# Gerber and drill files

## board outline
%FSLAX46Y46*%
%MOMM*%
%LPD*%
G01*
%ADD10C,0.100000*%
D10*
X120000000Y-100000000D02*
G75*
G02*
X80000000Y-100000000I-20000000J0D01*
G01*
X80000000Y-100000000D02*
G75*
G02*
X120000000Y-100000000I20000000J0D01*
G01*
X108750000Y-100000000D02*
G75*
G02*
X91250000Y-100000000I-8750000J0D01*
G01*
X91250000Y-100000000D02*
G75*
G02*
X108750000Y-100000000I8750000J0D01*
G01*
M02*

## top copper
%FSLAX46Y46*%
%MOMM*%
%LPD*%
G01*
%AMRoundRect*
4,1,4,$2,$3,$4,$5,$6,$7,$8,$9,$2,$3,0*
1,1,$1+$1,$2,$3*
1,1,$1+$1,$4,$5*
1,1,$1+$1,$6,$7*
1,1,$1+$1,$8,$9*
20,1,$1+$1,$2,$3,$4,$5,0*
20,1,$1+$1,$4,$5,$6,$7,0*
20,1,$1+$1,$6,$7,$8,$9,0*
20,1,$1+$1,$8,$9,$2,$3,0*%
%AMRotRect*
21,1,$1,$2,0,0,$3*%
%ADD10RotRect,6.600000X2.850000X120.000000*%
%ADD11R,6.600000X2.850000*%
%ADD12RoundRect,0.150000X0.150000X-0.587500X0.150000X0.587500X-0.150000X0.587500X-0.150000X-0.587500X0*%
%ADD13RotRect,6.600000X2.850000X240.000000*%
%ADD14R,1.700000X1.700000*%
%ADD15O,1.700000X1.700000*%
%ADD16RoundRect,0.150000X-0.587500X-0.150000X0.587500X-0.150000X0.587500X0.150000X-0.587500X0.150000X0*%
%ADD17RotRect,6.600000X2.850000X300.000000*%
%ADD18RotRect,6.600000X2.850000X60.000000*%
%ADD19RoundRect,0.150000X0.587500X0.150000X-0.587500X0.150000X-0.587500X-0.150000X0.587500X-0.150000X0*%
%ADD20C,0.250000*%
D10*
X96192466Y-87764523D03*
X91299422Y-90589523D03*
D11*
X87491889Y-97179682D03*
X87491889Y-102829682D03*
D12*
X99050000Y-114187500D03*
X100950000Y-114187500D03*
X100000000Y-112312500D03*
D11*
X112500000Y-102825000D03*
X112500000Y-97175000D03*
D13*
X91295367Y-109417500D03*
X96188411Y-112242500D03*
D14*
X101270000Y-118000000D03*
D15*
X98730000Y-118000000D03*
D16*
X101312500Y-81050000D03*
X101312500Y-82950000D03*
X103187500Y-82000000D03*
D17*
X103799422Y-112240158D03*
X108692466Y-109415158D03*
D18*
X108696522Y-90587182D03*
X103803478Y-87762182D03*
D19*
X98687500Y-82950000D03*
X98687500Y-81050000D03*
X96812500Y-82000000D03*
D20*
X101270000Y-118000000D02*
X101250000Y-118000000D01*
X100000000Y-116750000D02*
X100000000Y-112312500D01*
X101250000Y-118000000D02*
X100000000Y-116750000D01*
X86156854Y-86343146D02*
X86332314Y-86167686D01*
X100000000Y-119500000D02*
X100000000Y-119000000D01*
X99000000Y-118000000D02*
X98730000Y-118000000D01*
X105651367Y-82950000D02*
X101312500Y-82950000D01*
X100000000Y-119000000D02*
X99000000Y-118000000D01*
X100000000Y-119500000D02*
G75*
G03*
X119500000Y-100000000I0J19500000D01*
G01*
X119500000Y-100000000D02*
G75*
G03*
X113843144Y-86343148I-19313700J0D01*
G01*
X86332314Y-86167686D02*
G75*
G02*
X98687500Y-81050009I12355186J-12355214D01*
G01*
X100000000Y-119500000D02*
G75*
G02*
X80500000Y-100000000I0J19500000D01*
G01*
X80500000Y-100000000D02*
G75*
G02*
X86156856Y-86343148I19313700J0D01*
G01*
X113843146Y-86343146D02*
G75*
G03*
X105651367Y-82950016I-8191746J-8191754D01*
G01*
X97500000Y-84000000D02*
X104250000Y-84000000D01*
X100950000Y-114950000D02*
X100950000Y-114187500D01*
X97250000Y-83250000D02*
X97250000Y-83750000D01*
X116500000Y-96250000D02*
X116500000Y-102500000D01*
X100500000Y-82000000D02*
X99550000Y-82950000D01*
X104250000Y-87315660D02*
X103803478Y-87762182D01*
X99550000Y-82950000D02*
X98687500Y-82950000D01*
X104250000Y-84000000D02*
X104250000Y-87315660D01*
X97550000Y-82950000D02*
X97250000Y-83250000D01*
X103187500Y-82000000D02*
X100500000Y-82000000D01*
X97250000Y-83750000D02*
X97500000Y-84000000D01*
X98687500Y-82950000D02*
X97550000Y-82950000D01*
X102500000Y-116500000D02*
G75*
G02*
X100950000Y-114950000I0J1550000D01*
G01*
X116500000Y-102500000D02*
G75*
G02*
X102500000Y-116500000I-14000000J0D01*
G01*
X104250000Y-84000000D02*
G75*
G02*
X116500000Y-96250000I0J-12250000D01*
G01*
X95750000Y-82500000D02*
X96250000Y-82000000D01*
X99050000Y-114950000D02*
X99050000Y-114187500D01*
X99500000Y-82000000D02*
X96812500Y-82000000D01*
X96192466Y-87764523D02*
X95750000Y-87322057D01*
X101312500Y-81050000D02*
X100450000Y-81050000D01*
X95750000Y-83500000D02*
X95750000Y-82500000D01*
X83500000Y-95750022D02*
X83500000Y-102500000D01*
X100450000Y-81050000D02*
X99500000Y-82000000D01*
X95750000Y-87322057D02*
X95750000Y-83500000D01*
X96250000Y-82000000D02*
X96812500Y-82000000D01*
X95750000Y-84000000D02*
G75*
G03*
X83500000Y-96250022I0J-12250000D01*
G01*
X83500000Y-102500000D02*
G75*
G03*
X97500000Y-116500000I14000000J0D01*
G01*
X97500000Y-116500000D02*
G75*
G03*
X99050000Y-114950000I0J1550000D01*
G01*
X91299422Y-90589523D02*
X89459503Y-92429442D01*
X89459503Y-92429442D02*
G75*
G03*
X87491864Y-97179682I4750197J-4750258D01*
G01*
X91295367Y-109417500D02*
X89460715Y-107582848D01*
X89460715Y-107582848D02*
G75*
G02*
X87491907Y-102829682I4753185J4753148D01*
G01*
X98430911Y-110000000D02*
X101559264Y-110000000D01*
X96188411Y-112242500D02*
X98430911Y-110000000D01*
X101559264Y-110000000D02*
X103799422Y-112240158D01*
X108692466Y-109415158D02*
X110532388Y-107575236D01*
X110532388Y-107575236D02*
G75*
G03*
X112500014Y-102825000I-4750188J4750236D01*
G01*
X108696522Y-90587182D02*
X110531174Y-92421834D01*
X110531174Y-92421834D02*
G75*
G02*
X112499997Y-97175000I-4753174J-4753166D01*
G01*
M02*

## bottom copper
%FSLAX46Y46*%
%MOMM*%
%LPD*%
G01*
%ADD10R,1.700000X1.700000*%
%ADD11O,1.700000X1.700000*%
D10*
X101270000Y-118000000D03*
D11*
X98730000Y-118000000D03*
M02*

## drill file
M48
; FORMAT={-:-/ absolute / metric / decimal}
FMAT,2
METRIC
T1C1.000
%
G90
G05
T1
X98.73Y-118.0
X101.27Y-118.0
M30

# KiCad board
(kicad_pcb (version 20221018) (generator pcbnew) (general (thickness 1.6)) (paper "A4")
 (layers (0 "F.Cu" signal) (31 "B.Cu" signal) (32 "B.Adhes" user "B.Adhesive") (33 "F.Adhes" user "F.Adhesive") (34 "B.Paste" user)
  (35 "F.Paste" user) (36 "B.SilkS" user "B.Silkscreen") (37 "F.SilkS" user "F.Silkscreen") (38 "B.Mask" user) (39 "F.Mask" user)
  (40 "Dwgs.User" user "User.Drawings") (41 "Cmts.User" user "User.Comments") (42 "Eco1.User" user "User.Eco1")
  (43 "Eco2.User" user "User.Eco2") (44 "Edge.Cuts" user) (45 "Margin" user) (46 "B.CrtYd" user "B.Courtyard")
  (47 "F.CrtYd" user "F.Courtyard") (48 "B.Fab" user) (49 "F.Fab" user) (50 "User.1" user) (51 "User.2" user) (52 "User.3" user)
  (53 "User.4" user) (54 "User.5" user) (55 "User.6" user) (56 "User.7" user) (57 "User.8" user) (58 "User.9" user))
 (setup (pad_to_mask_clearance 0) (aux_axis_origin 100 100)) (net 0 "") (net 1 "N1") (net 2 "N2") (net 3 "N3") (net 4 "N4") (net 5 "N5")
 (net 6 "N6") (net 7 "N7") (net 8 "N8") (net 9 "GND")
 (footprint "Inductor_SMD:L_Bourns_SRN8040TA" (layer "F.Cu") (at 93.745944 89.177023 -150)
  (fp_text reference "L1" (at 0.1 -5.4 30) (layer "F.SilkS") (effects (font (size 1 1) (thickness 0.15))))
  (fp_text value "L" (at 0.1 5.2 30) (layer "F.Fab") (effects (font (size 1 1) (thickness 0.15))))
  (pad "1" smd rect (at -2.825 0 120) (size 6.6 2.85) (layers "F.Cu" "F.Paste" "F.Mask") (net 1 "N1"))
  (pad "2" smd rect (at 2.825 0 120) (size 6.6 2.85) (layers "F.Cu" "F.Paste" "F.Mask") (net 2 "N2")))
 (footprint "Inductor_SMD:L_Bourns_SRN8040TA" (layer "F.Cu") (at 87.491889 100.004682 -90)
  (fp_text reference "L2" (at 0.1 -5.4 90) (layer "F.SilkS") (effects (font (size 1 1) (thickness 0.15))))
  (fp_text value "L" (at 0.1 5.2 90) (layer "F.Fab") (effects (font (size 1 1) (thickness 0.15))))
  (pad "1" smd rect (at -2.825 0 180) (size 6.6 2.85) (layers "F.Cu" "F.Paste" "F.Mask") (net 2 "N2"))
  (pad "2" smd rect (at 2.825 0 180) (size 6.6 2.85) (layers "F.Cu" "F.Paste" "F.Mask") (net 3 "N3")))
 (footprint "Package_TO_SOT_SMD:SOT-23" (layer "F.Cu") (at 100 113.25 90)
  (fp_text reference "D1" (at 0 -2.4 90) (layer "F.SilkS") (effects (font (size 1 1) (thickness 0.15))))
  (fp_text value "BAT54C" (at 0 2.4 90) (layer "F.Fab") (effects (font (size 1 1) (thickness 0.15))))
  (pad "1" smd roundrect (at -0.9375 -0.95 90) (size 1.475 0.6) (layers "F.Cu" "F.Paste" "F.Mask") (roundrect_rratio 0.25) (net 1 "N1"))
  (pad "2" smd roundrect (at -0.9375 0.95 90) (size 1.475 0.6) (layers "F.Cu" "F.Paste" "F.Mask") (roundrect_rratio 0.25) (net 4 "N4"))
  (pad "3" smd roundrect (at 0.9375 0 90) (size 1.475 0.6) (layers "F.Cu" "F.Paste" "F.Mask") (roundrect_rratio 0.25) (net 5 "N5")))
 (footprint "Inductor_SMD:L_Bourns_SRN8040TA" (layer "F.Cu") (at 112.5 100 90)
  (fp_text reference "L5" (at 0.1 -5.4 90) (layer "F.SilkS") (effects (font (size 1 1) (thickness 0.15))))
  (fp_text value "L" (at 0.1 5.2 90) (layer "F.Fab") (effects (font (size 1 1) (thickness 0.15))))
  (pad "1" smd rect (at -2.825 0) (size 6.6 2.85) (layers "F.Cu" "F.Paste" "F.Mask") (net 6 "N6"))
  (pad "2" smd rect (at 2.825 0) (size 6.6 2.85) (layers "F.Cu" "F.Paste" "F.Mask") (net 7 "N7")))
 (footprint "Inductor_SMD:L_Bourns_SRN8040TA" (layer "F.Cu") (at 93.741889 110.83 -30)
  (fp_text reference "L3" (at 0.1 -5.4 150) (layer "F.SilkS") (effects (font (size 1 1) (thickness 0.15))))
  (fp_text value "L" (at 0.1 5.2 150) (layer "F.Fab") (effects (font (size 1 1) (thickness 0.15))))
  (pad "1" smd rect (at -2.825 0 240) (size 6.6 2.85) (layers "F.Cu" "F.Paste" "F.Mask") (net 3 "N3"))
  (pad "2" smd rect (at 2.825 0 240) (size 6.6 2.85) (layers "F.Cu" "F.Paste" "F.Mask") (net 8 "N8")))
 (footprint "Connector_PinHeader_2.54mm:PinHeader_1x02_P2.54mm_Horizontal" (layer "F.Cu") (at 101.27 118 -90)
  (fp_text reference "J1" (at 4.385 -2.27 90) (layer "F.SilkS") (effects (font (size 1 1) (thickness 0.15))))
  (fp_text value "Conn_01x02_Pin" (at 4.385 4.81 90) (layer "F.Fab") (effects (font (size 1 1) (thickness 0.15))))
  (pad "1" thru_hole rect (at 0 0 270) (size 1.7 1.7) (drill 1) (layers "*.Cu" "*.Mask") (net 5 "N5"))
  (pad "2" thru_hole oval (at 0 2.54 270) (size 1.7 1.7) (drill 1) (layers "*.Cu" "*.Mask") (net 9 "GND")))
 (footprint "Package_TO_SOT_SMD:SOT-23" (layer "F.Cu") (at 102.25 82)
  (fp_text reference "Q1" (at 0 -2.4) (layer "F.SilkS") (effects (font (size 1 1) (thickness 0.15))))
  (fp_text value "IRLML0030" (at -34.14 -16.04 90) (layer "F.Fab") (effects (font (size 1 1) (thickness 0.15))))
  (pad "1" smd roundrect (at -0.9375 -0.95) (size 1.475 0.6) (layers "F.Cu" "F.Paste" "F.Mask") (roundrect_rratio 0.25) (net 1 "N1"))
  (pad "2" smd roundrect (at -0.9375 0.95) (size 1.475 0.6) (layers "F.Cu" "F.Paste" "F.Mask") (roundrect_rratio 0.25) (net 9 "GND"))
  (pad "3" smd roundrect (at 0.9375 0) (size 1.475 0.6) (layers "F.Cu" "F.Paste" "F.Mask") (roundrect_rratio 0.25) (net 4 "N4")))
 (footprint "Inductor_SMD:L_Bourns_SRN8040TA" (layer "F.Cu") (at 106.245944 110.827658 30)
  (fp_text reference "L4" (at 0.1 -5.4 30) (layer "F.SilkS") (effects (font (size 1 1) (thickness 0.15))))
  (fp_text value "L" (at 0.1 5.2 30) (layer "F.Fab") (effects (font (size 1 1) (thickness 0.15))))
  (pad "1" smd rect (at -2.825 0 300) (size 6.6 2.85) (layers "F.Cu" "F.Paste" "F.Mask") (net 8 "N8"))
  (pad "2" smd rect (at 2.825 0 300) (size 6.6 2.85) (layers "F.Cu" "F.Paste" "F.Mask") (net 6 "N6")))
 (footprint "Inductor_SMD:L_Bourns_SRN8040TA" (layer "F.Cu") (at 106.25 89.174682 150)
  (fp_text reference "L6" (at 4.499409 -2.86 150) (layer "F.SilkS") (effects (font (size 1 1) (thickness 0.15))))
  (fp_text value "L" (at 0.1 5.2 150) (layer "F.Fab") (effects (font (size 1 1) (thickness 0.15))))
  (pad "1" smd rect (at -2.825 0 60) (size 6.6 2.85) (layers "F.Cu" "F.Paste" "F.Mask") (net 7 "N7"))
  (pad "2" smd rect (at 2.825 0 60) (size 6.6 2.85) (layers "F.Cu" "F.Paste" "F.Mask") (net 4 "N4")))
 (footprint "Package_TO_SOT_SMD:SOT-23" (layer "F.Cu") (at 97.75 82 180)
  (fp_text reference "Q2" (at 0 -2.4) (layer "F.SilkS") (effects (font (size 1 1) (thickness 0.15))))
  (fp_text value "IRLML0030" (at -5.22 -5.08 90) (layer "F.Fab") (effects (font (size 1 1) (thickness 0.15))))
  (pad "1" smd roundrect (at -0.9375 -0.95 180) (size 1.475 0.6) (layers "F.Cu" "F.Paste" "F.Mask") (roundrect_rratio 0.25) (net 4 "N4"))
  (pad "2" smd roundrect (at -0.9375 0.95 180) (size 1.475 0.6) (layers "F.Cu" "F.Paste" "F.Mask") (roundrect_rratio 0.25) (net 9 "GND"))
  (pad "3" smd roundrect (at 0.9375 0 180) (size 1.475 0.6) (layers "F.Cu" "F.Paste" "F.Mask") (roundrect_rratio 0.25) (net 1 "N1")))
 (gr_circle (center 100 100) (end 80 100) (stroke (width 0.1) (type default)) (fill none) (layer "Edge.Cuts"))
 (gr_circle (center 100 100) (end 108.75 100) (stroke (width 0.1) (type default)) (fill none) (layer "Edge.Cuts"))
 (segment (start 101.27 118) (end 101.25 118) (width 0.25) (layer "F.Cu") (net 5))
 (segment (start 100 116.75) (end 100 112.3125) (width 0.25) (layer "F.Cu") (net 5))
 (segment (start 101.25 118) (end 100 116.75) (width 0.25) (layer "F.Cu") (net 5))
 (segment (start 86.156854 86.343146) (end 86.332314 86.167686) (width 0.25) (layer "F.Cu") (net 9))
 (segment (start 100 119.5) (end 100 119) (width 0.25) (layer "F.Cu") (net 9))
 (segment (start 99 118) (end 98.73 118) (width 0.25) (layer "F.Cu") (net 9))
 (segment (start 105.651367 82.95) (end 101.3125 82.95) (width 0.25) (layer "F.Cu") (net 9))
 (segment (start 100 119) (end 99 118) (width 0.25) (layer "F.Cu") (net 9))
 (arc (start 100 119.5) (mid 113.788582 113.788582) (end 119.5 100) (width 0.25) (layer "F.Cu") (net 9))
 (arc (start 119.5 100) (mid 118.029832 92.608964) (end 113.843146 86.343146) (width 0.25) (layer "F.Cu") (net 9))
 (arc (start 86.332314 86.167686) (mid 92.000921 82.380044) (end 98.6875 81.05) (width 0.25) (layer "F.Cu") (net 9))
 (arc (start 100 119.5) (mid 86.211418 113.788582) (end 80.5 100) (width 0.25) (layer "F.Cu") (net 9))
 (arc (start 80.5 100) (mid 81.970168 92.608964) (end 86.156854 86.343146) (width 0.25) (layer "F.Cu") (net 9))
 (arc (start 113.843146 86.343146) (mid 110.084726 83.83185) (end 105.651367 82.95) (width 0.25) (layer "F.Cu") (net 9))
 (segment (start 97.5 84) (end 104.25 84) (width 0.25) (layer "F.Cu") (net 4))
 (segment (start 100.95 114.95) (end 100.95 114.1875) (width 0.25) (layer "F.Cu") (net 4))
 (segment (start 97.25 83.25) (end 97.25 83.75) (width 0.25) (layer "F.Cu") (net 4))
 (segment (start 116.5 96.25) (end 116.5 102.5) (width 0.25) (layer "F.Cu") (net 4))
 (segment (start 100.5 82) (end 99.55 82.95) (width 0.25) (layer "F.Cu") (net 4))
 (segment (start 104.25 87.31566) (end 103.803478 87.762182) (width 0.25) (layer "F.Cu") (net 4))
 (segment (start 99.55 82.95) (end 98.6875 82.95) (width 0.25) (layer "F.Cu") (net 4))
 (segment (start 104.25 84) (end 104.25 87.31566) (width 0.25) (layer "F.Cu") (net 4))
 (segment (start 97.55 82.95) (end 97.25 83.25) (width 0.25) (layer "F.Cu") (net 4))
 (segment (start 103.1875 82) (end 100.5 82) (width 0.25) (layer "F.Cu") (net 4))
 (segment (start 97.25 83.75) (end 97.5 84) (width 0.25) (layer "F.Cu") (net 4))
 (segment (start 98.6875 82.95) (end 97.55 82.95) (width 0.25) (layer "F.Cu") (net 4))
 (arc (start 102.5 116.5) (mid 101.403984 116.046016) (end 100.95 114.95) (width 0.25) (layer "F.Cu") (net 4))
 (arc (start 116.5 102.5) (mid 112.399495 112.399495) (end 102.5 116.5) (width 0.25) (layer "F.Cu") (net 4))
 (arc (start 104.25 84) (mid 112.912058 87.587942) (end 116.5 96.25) (width 0.25) (layer "F.Cu") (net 4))
 (segment (start 95.75 82.5) (end 96.25 82) (width 0.25) (layer "F.Cu") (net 1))
 (segment (start 99.05 114.95) (end 99.05 114.1875) (width 0.25) (layer "F.Cu") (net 1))
 (segment (start 99.5 82) (end 96.8125 82) (width 0.25) (layer "F.Cu") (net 1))
 (segment (start 96.192466 87.764523) (end 95.75 87.322057) (width 0.25) (layer "F.Cu") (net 1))
 (segment (start 101.3125 81.05) (end 100.45 81.05) (width 0.25) (layer "F.Cu") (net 1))
 (segment (start 95.75 83.5) (end 95.75 82.5) (width 0.25) (layer "F.Cu") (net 1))
 (segment (start 83.5 95.750022) (end 83.5 102.5) (width 0.25) (layer "F.Cu") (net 1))
 (segment (start 100.45 81.05) (end 99.5 82) (width 0.25) (layer "F.Cu") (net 1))
 (segment (start 95.75 87.322057) (end 95.75 83.5) (width 0.25) (layer "F.Cu") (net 1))
 (segment (start 96.25 82) (end 96.8125 82) (width 0.25) (layer "F.Cu") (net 1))
 (arc (start 95.75 84) (mid 87.087948 87.587948) (end 83.5 96.250022) (width 0.25) (layer "F.Cu") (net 1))
 (arc (start 83.5 102.5) (mid 87.600505 112.399495) (end 97.5 116.5) (width 0.25) (layer "F.Cu") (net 1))
 (arc (start 97.5 116.5) (mid 98.596016 116.046016) (end 99.05 114.95) (width 0.25) (layer "F.Cu") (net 1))
 (segment (start 91.299422 90.589523) (end 89.459503 92.429442) (width 0.25) (layer "F.Cu") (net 2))
 (arc (start 89.459503 92.429442) (mid 88.003255 94.60887) (end 87.491889 97.179682) (width 0.25) (layer "F.Cu") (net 2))
 (segment (start 91.295367 109.4175) (end 89.460715 107.582848) (width 0.25) (layer "F.Cu") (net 3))
 (arc (start 89.460715 107.582848) (mid 88.003571 105.402078) (end 87.491889 102.829682) (width 0.25) (layer "F.Cu") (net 3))
 (segment (start 98.430911 110) (end 101.559264 110) (width 0.25) (layer "F.Cu") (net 8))
 (segment (start 96.188411 112.2425) (end 98.430911 110) (width 0.25) (layer "F.Cu") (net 8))
 (segment (start 101.559264 110) (end 103.799422 112.240158) (width 0.25) (layer "F.Cu") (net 8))
 (segment (start 108.692466 109.415158) (end 110.532388 107.575236) (width 0.25) (layer "F.Cu") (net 6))
 (arc (start 110.532388 107.575236) (mid 111.988634 105.39581) (end 112.5 102.825) (width 0.25) (layer "F.Cu") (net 6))
 (segment (start 108.696522 90.587182) (end 110.531174 92.421834) (width 0.25) (layer "F.Cu") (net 7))
 (arc (start 110.531174 92.421834) (mid 111.988318 94.602604) (end 112.5 97.175) (width 0.25) (layer "F.Cu") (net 7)))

